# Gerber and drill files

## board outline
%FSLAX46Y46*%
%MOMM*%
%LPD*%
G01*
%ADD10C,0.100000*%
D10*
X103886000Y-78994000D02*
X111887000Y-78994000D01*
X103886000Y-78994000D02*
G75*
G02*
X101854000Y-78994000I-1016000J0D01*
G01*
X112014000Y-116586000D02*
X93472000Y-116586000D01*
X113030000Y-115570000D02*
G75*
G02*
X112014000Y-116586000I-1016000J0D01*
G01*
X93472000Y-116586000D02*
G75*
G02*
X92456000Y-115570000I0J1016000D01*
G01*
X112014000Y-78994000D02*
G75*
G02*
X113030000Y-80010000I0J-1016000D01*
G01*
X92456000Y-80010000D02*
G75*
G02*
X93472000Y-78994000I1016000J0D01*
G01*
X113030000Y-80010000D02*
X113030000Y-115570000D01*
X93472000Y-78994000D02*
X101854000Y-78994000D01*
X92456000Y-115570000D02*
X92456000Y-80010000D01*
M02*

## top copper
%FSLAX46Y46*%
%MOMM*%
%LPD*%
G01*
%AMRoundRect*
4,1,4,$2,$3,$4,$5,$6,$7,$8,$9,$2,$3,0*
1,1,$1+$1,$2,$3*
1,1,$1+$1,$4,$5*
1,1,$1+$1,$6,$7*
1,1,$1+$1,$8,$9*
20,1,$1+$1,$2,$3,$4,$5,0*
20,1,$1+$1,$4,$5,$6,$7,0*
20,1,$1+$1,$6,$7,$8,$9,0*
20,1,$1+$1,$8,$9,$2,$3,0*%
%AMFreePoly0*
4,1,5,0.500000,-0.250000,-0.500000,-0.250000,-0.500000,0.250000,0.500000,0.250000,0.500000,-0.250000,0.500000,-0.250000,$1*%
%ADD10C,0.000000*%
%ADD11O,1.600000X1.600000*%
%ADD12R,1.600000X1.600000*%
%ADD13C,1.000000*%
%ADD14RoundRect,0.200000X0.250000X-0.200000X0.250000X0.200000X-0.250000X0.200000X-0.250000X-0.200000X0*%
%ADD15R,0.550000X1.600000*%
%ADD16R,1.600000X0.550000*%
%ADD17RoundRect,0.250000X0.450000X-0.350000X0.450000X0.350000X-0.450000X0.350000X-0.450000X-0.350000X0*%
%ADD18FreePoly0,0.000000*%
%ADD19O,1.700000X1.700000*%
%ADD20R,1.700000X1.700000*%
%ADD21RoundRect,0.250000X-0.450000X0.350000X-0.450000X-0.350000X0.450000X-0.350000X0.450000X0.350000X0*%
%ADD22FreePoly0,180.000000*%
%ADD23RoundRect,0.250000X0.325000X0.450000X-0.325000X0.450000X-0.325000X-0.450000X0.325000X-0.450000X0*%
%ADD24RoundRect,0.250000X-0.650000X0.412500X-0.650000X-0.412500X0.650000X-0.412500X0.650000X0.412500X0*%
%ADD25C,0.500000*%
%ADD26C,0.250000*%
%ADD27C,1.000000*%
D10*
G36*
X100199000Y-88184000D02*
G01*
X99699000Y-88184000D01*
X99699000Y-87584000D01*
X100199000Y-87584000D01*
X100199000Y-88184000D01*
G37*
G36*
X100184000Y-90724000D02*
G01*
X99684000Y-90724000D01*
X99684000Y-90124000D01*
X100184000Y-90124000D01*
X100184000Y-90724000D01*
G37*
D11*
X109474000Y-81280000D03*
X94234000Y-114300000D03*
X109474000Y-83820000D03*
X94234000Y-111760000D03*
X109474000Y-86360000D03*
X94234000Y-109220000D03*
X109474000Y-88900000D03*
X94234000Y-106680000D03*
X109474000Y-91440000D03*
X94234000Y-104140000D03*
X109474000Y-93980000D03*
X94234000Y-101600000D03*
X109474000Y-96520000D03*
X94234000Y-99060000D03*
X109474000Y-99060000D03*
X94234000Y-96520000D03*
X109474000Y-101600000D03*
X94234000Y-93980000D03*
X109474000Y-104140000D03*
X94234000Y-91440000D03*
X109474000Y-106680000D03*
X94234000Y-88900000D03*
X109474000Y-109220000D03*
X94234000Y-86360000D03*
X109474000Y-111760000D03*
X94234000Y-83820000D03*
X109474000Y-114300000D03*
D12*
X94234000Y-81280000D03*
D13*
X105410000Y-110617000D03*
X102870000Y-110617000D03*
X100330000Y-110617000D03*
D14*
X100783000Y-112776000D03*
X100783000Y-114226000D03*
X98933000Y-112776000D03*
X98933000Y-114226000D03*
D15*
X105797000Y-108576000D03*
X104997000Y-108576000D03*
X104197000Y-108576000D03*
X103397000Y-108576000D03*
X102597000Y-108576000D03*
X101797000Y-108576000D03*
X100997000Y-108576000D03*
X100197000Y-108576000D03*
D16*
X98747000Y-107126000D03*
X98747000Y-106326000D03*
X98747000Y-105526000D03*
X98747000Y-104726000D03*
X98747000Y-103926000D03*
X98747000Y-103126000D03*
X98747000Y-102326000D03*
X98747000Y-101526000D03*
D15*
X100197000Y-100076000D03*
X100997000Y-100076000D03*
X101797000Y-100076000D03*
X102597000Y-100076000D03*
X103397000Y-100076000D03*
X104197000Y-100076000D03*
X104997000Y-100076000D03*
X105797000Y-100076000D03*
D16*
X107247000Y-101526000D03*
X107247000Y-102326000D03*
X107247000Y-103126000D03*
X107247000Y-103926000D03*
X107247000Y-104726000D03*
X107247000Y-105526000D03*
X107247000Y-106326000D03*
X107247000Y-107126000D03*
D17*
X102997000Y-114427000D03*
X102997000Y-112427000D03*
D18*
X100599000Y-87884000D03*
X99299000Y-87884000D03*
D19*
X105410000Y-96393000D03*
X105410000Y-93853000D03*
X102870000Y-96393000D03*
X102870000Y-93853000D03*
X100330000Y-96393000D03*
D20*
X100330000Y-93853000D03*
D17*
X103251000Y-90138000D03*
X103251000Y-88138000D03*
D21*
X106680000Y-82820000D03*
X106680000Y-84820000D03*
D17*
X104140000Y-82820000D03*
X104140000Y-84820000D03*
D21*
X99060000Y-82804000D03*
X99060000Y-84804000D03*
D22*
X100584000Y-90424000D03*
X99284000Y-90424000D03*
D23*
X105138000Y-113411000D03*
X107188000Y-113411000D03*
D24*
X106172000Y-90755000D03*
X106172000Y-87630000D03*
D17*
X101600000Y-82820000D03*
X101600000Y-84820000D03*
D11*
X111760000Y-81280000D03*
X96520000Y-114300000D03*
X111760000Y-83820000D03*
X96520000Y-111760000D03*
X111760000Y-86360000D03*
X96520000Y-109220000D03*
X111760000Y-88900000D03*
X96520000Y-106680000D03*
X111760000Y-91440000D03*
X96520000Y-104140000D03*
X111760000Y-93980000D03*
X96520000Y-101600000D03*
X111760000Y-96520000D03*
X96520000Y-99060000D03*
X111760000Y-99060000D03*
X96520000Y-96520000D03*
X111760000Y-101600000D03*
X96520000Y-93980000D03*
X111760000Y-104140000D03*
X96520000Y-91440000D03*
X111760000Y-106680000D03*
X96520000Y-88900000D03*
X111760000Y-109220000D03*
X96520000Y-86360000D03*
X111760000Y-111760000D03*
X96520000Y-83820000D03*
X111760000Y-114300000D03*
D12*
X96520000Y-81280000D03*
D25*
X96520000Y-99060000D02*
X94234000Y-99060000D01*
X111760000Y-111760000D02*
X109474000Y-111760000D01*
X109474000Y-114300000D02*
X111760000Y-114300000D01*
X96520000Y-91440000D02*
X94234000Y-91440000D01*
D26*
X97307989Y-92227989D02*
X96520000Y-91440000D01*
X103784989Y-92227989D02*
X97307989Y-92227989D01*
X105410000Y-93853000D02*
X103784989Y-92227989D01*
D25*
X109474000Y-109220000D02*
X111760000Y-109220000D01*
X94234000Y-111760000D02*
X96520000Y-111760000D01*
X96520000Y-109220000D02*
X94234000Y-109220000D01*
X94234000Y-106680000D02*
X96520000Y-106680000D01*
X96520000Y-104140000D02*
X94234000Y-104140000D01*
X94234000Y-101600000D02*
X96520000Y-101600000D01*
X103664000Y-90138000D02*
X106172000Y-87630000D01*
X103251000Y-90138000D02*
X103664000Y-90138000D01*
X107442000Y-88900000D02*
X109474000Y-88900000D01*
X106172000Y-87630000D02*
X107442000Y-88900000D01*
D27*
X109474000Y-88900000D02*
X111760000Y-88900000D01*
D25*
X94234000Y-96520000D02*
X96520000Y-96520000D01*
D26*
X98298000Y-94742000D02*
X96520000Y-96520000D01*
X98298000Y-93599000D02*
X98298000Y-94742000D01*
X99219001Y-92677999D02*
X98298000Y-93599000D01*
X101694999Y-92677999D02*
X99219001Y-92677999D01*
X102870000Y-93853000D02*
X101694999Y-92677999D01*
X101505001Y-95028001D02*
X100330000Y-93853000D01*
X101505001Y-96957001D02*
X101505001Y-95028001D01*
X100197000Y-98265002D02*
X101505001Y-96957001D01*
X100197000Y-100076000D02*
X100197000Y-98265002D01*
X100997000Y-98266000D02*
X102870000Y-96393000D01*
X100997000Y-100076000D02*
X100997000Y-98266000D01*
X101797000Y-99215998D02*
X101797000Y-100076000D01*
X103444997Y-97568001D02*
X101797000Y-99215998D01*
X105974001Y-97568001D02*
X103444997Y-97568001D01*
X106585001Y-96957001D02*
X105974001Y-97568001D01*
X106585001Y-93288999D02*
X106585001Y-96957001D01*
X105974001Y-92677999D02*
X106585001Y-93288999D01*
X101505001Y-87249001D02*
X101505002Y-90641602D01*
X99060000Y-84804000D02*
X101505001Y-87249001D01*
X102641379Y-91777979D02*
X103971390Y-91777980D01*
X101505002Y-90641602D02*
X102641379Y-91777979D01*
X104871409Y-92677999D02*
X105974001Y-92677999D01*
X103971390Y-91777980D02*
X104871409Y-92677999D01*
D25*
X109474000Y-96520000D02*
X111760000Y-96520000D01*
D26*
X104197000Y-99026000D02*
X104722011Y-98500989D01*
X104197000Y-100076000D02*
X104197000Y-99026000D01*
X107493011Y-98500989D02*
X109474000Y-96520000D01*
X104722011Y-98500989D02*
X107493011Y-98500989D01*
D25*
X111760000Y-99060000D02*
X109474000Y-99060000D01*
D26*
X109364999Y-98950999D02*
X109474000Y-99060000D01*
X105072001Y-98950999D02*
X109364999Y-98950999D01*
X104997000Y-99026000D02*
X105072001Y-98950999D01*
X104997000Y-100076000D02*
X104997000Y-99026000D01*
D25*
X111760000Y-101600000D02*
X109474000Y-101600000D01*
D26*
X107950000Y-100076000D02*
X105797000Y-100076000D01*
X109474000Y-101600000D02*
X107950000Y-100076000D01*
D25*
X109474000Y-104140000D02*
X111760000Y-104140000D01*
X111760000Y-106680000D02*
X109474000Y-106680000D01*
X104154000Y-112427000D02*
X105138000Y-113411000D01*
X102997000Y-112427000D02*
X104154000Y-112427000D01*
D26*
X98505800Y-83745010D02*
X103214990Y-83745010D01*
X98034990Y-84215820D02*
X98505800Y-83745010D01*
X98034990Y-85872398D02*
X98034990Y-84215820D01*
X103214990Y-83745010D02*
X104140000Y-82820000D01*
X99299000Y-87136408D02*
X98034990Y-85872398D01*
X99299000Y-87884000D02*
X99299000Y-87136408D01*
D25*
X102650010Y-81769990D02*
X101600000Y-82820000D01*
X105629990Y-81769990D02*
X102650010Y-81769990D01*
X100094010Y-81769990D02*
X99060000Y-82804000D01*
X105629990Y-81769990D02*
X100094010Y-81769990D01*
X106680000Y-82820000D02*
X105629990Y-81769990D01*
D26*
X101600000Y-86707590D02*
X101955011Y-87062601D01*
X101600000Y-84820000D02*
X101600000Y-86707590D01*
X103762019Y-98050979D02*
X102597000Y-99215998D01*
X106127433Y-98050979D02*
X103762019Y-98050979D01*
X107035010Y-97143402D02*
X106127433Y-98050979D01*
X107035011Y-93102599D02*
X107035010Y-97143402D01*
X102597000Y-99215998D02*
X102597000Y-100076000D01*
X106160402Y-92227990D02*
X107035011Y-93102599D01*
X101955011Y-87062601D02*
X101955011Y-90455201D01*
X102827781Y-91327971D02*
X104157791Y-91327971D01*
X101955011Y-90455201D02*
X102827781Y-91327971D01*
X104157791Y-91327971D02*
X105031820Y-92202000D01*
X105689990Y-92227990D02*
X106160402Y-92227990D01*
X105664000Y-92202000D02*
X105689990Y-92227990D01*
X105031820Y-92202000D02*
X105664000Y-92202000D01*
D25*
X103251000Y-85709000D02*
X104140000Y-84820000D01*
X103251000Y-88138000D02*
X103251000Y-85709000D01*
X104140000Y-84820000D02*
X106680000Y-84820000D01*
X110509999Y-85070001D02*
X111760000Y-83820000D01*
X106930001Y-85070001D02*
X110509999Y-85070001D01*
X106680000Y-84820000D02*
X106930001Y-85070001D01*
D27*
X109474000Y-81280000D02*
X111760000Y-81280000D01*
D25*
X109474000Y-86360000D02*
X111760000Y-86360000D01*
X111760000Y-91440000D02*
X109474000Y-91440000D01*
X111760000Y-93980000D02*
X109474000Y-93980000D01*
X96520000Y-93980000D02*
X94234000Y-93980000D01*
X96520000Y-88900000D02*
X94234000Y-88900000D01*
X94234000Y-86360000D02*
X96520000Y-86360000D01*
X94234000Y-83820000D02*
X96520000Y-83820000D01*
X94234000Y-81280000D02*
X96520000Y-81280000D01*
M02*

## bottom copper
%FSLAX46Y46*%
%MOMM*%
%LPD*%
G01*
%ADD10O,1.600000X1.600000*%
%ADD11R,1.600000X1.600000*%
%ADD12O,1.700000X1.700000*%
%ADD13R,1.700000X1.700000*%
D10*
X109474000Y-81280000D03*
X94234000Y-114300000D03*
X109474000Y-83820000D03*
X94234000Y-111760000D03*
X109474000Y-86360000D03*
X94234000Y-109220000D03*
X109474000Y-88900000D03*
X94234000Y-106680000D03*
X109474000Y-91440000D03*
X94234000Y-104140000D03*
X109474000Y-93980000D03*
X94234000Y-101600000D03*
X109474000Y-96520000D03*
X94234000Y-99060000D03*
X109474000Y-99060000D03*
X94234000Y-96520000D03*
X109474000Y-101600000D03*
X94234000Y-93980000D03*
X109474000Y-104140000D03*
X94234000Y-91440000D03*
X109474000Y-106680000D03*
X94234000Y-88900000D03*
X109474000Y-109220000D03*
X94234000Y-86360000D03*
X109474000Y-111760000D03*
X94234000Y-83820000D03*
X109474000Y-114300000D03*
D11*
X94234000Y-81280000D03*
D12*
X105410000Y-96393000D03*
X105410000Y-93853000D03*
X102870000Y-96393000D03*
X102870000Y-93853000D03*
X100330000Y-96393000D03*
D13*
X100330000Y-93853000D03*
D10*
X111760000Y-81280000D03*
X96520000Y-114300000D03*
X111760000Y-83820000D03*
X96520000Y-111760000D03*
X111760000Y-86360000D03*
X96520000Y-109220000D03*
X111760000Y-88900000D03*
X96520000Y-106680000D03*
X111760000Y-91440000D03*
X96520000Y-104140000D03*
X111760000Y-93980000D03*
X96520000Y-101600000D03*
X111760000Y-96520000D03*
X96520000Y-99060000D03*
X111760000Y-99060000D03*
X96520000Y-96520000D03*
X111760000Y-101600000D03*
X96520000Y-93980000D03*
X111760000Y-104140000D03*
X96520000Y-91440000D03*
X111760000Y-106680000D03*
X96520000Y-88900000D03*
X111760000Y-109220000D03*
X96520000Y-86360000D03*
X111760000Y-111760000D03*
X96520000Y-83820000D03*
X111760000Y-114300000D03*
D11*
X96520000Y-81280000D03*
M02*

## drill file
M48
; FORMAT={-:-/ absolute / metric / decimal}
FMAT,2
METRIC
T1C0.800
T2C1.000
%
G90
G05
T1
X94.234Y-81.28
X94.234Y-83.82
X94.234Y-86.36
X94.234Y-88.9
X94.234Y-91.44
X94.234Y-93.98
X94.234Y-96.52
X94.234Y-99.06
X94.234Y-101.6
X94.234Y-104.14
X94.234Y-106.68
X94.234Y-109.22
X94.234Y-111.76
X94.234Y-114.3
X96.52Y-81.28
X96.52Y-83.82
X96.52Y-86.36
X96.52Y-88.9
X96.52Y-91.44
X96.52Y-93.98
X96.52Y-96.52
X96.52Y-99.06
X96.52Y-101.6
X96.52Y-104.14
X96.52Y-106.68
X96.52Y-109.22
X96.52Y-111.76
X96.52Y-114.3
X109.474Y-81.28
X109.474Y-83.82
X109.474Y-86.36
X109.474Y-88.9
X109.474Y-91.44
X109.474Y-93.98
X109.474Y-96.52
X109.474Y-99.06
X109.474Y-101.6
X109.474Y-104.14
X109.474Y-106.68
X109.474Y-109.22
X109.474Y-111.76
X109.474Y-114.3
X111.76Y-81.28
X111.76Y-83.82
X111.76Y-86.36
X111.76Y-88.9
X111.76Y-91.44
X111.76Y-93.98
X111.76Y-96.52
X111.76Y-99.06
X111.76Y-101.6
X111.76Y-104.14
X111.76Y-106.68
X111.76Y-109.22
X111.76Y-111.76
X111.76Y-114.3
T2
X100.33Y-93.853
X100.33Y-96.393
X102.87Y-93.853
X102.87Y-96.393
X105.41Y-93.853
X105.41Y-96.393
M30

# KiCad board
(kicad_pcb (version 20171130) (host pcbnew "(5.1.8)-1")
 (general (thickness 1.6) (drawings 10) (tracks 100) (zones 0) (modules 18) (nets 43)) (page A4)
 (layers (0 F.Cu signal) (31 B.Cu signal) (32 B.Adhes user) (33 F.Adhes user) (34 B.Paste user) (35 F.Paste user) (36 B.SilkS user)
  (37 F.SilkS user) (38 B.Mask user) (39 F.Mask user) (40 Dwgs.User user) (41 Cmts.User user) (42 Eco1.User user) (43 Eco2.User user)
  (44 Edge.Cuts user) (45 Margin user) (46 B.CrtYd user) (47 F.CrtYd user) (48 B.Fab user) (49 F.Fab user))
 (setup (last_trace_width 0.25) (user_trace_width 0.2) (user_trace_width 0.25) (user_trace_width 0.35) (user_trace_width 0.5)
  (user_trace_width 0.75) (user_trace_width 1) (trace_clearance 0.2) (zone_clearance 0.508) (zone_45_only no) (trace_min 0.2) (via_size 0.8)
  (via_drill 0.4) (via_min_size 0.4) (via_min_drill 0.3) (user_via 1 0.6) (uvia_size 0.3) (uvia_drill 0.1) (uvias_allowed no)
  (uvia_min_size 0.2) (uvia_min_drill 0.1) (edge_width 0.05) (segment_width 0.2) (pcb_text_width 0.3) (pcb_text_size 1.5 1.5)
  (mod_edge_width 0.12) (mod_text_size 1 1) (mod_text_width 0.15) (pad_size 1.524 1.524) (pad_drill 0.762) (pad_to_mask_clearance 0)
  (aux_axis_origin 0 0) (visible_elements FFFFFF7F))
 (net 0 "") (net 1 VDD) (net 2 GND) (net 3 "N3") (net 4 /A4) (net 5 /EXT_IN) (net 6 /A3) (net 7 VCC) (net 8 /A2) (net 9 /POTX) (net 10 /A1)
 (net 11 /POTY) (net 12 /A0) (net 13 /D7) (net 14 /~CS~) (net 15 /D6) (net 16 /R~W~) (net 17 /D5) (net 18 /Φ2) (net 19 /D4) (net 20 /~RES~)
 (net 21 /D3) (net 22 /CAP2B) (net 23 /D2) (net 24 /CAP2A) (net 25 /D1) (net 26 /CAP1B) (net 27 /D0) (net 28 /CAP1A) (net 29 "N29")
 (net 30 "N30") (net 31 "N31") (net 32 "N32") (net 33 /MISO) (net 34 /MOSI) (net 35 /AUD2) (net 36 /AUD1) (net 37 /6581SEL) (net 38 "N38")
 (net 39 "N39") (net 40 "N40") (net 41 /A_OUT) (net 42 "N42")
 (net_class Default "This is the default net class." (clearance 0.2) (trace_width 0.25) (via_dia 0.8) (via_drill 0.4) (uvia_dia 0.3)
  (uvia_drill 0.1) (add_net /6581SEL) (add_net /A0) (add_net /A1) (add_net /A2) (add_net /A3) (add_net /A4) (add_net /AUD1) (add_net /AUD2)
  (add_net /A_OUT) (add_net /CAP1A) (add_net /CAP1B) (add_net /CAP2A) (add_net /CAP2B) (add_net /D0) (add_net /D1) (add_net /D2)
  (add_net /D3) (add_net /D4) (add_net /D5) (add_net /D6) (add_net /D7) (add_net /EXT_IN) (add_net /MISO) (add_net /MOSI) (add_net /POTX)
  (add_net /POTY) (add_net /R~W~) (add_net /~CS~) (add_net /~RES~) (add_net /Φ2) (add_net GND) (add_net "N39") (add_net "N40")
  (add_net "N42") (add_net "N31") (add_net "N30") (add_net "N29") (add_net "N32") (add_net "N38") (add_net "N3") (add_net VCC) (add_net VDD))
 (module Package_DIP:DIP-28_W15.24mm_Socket (layer F.Cu) (at 94.234 81.28)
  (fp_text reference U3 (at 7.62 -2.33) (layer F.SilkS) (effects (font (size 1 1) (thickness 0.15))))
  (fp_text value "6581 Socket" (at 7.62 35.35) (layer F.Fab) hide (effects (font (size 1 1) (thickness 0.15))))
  (pad 28 thru_hole oval (at 15.24 0) (size 1.6 1.6) (drill 0.8) (layers *.Cu *.Mask) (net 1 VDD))
  (pad 14 thru_hole oval (at 0 33.02) (size 1.6 1.6) (drill 0.8) (layers *.Cu *.Mask) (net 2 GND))
  (pad 27 thru_hole oval (at 15.24 2.54) (size 1.6 1.6) (drill 0.8) (layers *.Cu *.Mask) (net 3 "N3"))
  (pad 13 thru_hole oval (at 0 30.48) (size 1.6 1.6) (drill 0.8) (layers *.Cu *.Mask) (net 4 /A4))
  (pad 26 thru_hole oval (at 15.24 5.08) (size 1.6 1.6) (drill 0.8) (layers *.Cu *.Mask) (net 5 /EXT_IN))
  (pad 12 thru_hole oval (at 0 27.94) (size 1.6 1.6) (drill 0.8) (layers *.Cu *.Mask) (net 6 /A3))
  (pad 25 thru_hole oval (at 15.24 7.62) (size 1.6 1.6) (drill 0.8) (layers *.Cu *.Mask) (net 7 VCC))
  (pad 11 thru_hole oval (at 0 25.4) (size 1.6 1.6) (drill 0.8) (layers *.Cu *.Mask) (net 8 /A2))
  (pad 24 thru_hole oval (at 15.24 10.16) (size 1.6 1.6) (drill 0.8) (layers *.Cu *.Mask) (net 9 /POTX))
  (pad 10 thru_hole oval (at 0 22.86) (size 1.6 1.6) (drill 0.8) (layers *.Cu *.Mask) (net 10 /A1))
  (pad 23 thru_hole oval (at 15.24 12.7) (size 1.6 1.6) (drill 0.8) (layers *.Cu *.Mask) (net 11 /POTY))
  (pad 9 thru_hole oval (at 0 20.32) (size 1.6 1.6) (drill 0.8) (layers *.Cu *.Mask) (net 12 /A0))
  (pad 22 thru_hole oval (at 15.24 15.24) (size 1.6 1.6) (drill 0.8) (layers *.Cu *.Mask) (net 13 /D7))
  (pad 8 thru_hole oval (at 0 17.78) (size 1.6 1.6) (drill 0.8) (layers *.Cu *.Mask) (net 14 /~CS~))
  (pad 21 thru_hole oval (at 15.24 17.78) (size 1.6 1.6) (drill 0.8) (layers *.Cu *.Mask) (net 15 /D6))
  (pad 7 thru_hole oval (at 0 15.24) (size 1.6 1.6) (drill 0.8) (layers *.Cu *.Mask) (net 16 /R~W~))
  (pad 20 thru_hole oval (at 15.24 20.32) (size 1.6 1.6) (drill 0.8) (layers *.Cu *.Mask) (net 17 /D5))
  (pad 6 thru_hole oval (at 0 12.7) (size 1.6 1.6) (drill 0.8) (layers *.Cu *.Mask) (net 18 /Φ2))
  (pad 19 thru_hole oval (at 15.24 22.86) (size 1.6 1.6) (drill 0.8) (layers *.Cu *.Mask) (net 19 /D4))
  (pad 5 thru_hole oval (at 0 10.16) (size 1.6 1.6) (drill 0.8) (layers *.Cu *.Mask) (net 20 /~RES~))
  (pad 18 thru_hole oval (at 15.24 25.4) (size 1.6 1.6) (drill 0.8) (layers *.Cu *.Mask) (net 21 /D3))
  (pad 4 thru_hole oval (at 0 7.62) (size 1.6 1.6) (drill 0.8) (layers *.Cu *.Mask) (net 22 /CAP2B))
  (pad 17 thru_hole oval (at 15.24 27.94) (size 1.6 1.6) (drill 0.8) (layers *.Cu *.Mask) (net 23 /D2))
  (pad 3 thru_hole oval (at 0 5.08) (size 1.6 1.6) (drill 0.8) (layers *.Cu *.Mask) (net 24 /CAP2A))
  (pad 16 thru_hole oval (at 15.24 30.48) (size 1.6 1.6) (drill 0.8) (layers *.Cu *.Mask) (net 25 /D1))
  (pad 2 thru_hole oval (at 0 2.54) (size 1.6 1.6) (drill 0.8) (layers *.Cu *.Mask) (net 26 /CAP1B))
  (pad 15 thru_hole oval (at 15.24 33.02) (size 1.6 1.6) (drill 0.8) (layers *.Cu *.Mask) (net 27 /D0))
  (pad 1 thru_hole rect (at 0 0) (size 1.6 1.6) (drill 0.8) (layers *.Cu *.Mask) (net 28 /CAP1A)))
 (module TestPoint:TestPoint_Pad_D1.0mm (layer F.Cu) (at 105.41 110.617)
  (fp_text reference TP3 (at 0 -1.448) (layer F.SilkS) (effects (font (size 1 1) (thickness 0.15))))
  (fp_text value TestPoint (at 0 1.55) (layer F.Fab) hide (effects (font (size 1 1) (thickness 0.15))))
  (pad 1 smd circle (at 0 0) (size 1 1) (layers F.Cu F.Mask) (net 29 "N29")))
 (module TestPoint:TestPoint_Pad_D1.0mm (layer F.Cu) (at 102.87 110.617)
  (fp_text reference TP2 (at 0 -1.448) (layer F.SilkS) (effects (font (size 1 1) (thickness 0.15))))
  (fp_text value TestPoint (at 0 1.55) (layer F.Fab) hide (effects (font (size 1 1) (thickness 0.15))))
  (pad 1 smd circle (at 0 0) (size 1 1) (layers F.Cu F.Mask) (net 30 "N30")))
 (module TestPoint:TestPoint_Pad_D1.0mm (layer F.Cu) (at 100.33 110.617)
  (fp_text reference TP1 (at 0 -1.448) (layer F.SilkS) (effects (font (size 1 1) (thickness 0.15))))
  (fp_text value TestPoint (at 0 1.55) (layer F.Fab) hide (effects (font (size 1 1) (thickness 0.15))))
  (pad 1 smd circle (at 0 0) (size 1 1) (layers F.Cu F.Mask) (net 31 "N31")))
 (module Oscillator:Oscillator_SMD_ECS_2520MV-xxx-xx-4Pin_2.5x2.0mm (layer F.Cu) (at 99.858 113.501 90)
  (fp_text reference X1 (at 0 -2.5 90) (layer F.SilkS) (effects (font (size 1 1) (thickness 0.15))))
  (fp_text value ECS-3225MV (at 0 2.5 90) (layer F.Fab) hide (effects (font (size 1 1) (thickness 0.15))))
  (pad 3 smd roundrect (at 0.725 0.925 90) (size 0.8 0.9) (layers F.Cu F.Paste F.Mask) (roundrect_rratio 0.25) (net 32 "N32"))
  (pad 2 smd roundrect (at -0.725 0.925 90) (size 0.8 0.9) (layers F.Cu F.Paste F.Mask) (roundrect_rratio 0.25) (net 2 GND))
  (pad 4 smd roundrect (at 0.725 -0.925 90) (size 0.8 0.9) (layers F.Cu F.Paste F.Mask) (roundrect_rratio 0.25) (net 7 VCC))
  (pad 1 smd roundrect (at -0.725 -0.925 90) (size 0.8 0.9) (layers F.Cu F.Paste F.Mask) (roundrect_rratio 0.25) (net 7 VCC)))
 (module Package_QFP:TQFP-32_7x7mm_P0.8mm (layer F.Cu) (at 102.997 104.326 180)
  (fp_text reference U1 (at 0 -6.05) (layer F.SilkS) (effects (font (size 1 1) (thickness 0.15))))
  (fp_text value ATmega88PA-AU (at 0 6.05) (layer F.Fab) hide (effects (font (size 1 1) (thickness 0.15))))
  (pad 32 smd rect (at -2.8 -4.25 270) (size 1.6 0.55) (layers F.Cu F.Paste F.Mask) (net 14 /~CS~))
  (pad 31 smd rect (at -2 -4.25 270) (size 1.6 0.55) (layers F.Cu F.Paste F.Mask) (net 25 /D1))
  (pad 30 smd rect (at -1.2 -4.25 270) (size 1.6 0.55) (layers F.Cu F.Paste F.Mask) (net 27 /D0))
  (pad 29 smd rect (at -0.4 -4.25 270) (size 1.6 0.55) (layers F.Cu F.Paste F.Mask) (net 20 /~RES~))
  (pad 28 smd rect (at 0.4 -4.25 270) (size 1.6 0.55) (layers F.Cu F.Paste F.Mask) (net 23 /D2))
  (pad 27 smd rect (at 1.2 -4.25 270) (size 1.6 0.55) (layers F.Cu F.Paste F.Mask) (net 4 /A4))
  (pad 26 smd rect (at 2 -4.25 270) (size 1.6 0.55) (layers F.Cu F.Paste F.Mask) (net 6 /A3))
  (pad 25 smd rect (at 2.8 -4.25 270) (size 1.6 0.55) (layers F.Cu F.Paste F.Mask) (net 8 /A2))
  (pad 24 smd rect (at 4.25 -2.8 180) (size 1.6 0.55) (layers F.Cu F.Paste F.Mask) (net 10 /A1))
  (pad 23 smd rect (at 4.25 -2 180) (size 1.6 0.55) (layers F.Cu F.Paste F.Mask) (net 12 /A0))
  (pad 22 smd rect (at 4.25 -1.2 180) (size 1.6 0.55) (layers F.Cu F.Paste F.Mask) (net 30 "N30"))
  (pad 21 smd rect (at 4.25 -0.4 180) (size 1.6 0.55) (layers F.Cu F.Paste F.Mask) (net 2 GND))
  (pad 20 smd rect (at 4.25 0.4 180) (size 1.6 0.55) (layers F.Cu F.Paste F.Mask) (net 29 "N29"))
  (pad 19 smd rect (at 4.25 1.2 180) (size 1.6 0.55) (layers F.Cu F.Paste F.Mask) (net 31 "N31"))
  (pad 18 smd rect (at 4.25 2 180) (size 1.6 0.55) (layers F.Cu F.Paste F.Mask) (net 7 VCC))
  (pad 17 smd rect (at 4.25 2.8 180) (size 1.6 0.55) (layers F.Cu F.Paste F.Mask) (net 16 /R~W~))
  (pad 16 smd rect (at 2.8 4.25 270) (size 1.6 0.55) (layers F.Cu F.Paste F.Mask) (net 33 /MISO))
  (pad 15 smd rect (at 2 4.25 270) (size 1.6 0.55) (layers F.Cu F.Paste F.Mask) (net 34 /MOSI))
  (pad 14 smd rect (at 1.2 4.25 270) (size 1.6 0.55) (layers F.Cu F.Paste F.Mask) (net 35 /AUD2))
  (pad 13 smd rect (at 0.4 4.25 270) (size 1.6 0.55) (layers F.Cu F.Paste F.Mask) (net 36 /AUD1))
  (pad 12 smd rect (at -0.4 4.25 270) (size 1.6 0.55) (layers F.Cu F.Paste F.Mask) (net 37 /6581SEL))
  (pad 11 smd rect (at -1.2 4.25 270) (size 1.6 0.55) (layers F.Cu F.Paste F.Mask) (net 13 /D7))
  (pad 10 smd rect (at -2 4.25 270) (size 1.6 0.55) (layers F.Cu F.Paste F.Mask) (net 15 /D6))
  (pad 9 smd rect (at -2.8 4.25 270) (size 1.6 0.55) (layers F.Cu F.Paste F.Mask) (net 17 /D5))
  (pad 8 smd rect (at -4.25 2.8 180) (size 1.6 0.55) (layers F.Cu F.Paste F.Mask) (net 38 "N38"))
  (pad 7 smd rect (at -4.25 2 180) (size 1.6 0.55) (layers F.Cu F.Paste F.Mask) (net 32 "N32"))
  (pad 6 smd rect (at -4.25 1.2 180) (size 1.6 0.55) (layers F.Cu F.Paste F.Mask) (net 7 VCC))
  (pad 5 smd rect (at -4.25 0.4 180) (size 1.6 0.55) (layers F.Cu F.Paste F.Mask) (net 2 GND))
  (pad 4 smd rect (at -4.25 -0.4 180) (size 1.6 0.55) (layers F.Cu F.Paste F.Mask) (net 7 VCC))
  (pad 3 smd rect (at -4.25 -1.2 180) (size 1.6 0.55) (layers F.Cu F.Paste F.Mask) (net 2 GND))
  (pad 2 smd rect (at -4.25 -2 180) (size 1.6 0.55) (layers F.Cu F.Paste F.Mask) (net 19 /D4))
  (pad 1 smd rect (at -4.25 -2.8 180) (size 1.6 0.55) (layers F.Cu F.Paste F.Mask) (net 21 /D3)))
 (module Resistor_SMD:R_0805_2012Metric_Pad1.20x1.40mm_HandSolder (layer F.Cu) (at 102.997 113.427 90)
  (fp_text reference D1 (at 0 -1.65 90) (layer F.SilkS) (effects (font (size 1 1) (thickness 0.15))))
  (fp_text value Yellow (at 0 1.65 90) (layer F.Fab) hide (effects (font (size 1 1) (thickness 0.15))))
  (pad 1 smd roundrect (at -1 0 90) (size 1.2 1.4) (layers F.Cu F.Paste F.Mask) (roundrect_rratio 0.208333) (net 2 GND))
  (pad 2 smd roundrect (at 1 0 90) (size 1.2 1.4) (layers F.Cu F.Paste F.Mask) (roundrect_rratio 0.208333) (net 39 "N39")))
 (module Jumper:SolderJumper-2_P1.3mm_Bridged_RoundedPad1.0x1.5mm (layer F.Cu) (at 99.949 87.884)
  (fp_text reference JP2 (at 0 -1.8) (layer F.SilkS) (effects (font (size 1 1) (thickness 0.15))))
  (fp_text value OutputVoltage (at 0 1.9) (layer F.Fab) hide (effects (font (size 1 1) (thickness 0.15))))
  (fp_poly (pts (xy 0.25 -0.3) (xy -0.25 -0.3) (xy -0.25 0.3) (xy 0.25 0.3)) (layer F.Cu) (width 0))
  (pad 2 smd custom (at 0.65 0) (size 1 0.5) (layers F.Cu F.Mask) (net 2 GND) (zone_connect 2) (options (clearance outline) (anchor rect))
   (primitives))
  (pad 1 smd custom (at -0.65 0) (size 1 0.5) (layers F.Cu F.Mask) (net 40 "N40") (zone_connect 2)
   (options (clearance outline) (anchor rect)) (primitives)))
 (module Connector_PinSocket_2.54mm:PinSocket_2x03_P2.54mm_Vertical (layer F.Cu) (at 100.33 93.853 90)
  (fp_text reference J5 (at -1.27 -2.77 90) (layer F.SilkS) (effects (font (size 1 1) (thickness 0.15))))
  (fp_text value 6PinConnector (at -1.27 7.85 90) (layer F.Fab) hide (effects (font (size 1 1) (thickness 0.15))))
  (pad 6 thru_hole oval (at -2.54 5.08 90) (size 1.7 1.7) (drill 1) (layers *.Cu *.Mask) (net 2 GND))
  (pad 5 thru_hole oval (at 0 5.08 90) (size 1.7 1.7) (drill 1) (layers *.Cu *.Mask) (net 20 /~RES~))
  (pad 4 thru_hole oval (at -2.54 2.54 90) (size 1.7 1.7) (drill 1) (layers *.Cu *.Mask) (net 34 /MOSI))
  (pad 3 thru_hole oval (at 0 2.54 90) (size 1.7 1.7) (drill 1) (layers *.Cu *.Mask) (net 16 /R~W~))
  (pad 2 thru_hole oval (at -2.54 0 90) (size 1.7 1.7) (drill 1) (layers *.Cu *.Mask) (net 7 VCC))
  (pad 1 thru_hole rect (at 0 0 90) (size 1.7 1.7) (drill 1) (layers *.Cu *.Mask) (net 33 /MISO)))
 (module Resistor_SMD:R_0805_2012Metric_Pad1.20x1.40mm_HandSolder (layer F.Cu) (at 103.251 89.138 90)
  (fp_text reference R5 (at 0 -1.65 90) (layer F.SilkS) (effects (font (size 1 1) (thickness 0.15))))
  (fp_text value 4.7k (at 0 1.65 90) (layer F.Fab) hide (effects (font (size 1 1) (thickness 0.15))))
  (pad 1 smd roundrect (at -1 0 90) (size 1.2 1.4) (layers F.Cu F.Paste F.Mask) (roundrect_rratio 0.208333) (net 7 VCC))
  (pad 2 smd roundrect (at 1 0 90) (size 1.2 1.4) (layers F.Cu F.Paste F.Mask) (roundrect_rratio 0.208333) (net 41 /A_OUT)))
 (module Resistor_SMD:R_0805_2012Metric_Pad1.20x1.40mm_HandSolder (layer F.Cu) (at 106.68 83.82 270)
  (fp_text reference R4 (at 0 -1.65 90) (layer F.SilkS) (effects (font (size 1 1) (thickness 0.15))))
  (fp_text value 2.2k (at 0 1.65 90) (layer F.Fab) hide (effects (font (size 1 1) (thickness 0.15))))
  (pad 1 smd roundrect (at -1 0 270) (size 1.2 1.4) (layers F.Cu F.Paste F.Mask) (roundrect_rratio 0.208333) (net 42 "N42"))
  (pad 2 smd roundrect (at 1 0 270) (size 1.2 1.4) (layers F.Cu F.Paste F.Mask) (roundrect_rratio 0.208333) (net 41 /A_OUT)))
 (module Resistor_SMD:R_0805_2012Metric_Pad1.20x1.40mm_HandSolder (layer F.Cu) (at 104.14 83.82 90)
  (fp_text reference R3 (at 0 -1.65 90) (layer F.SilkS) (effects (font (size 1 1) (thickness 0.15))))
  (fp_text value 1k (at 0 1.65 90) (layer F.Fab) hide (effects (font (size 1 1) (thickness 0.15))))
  (pad 2 smd roundrect (at 1 0 90) (size 1.2 1.4) (layers F.Cu F.Paste F.Mask) (roundrect_rratio 0.208333) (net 40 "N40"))
  (pad 1 smd roundrect (at -1 0 90) (size 1.2 1.4) (layers F.Cu F.Paste F.Mask) (roundrect_rratio 0.208333) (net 41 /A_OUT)))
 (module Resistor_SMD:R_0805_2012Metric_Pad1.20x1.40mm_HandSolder (layer F.Cu) (at 99.06 83.804 270)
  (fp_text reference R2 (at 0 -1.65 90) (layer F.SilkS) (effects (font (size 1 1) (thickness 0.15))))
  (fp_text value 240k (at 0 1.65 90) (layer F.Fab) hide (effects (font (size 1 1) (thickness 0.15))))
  (pad 1 smd roundrect (at -1 0 270) (size 1.2 1.4) (layers F.Cu F.Paste F.Mask) (roundrect_rratio 0.208333) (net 42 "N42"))
  (pad 2 smd roundrect (at 1 0 270) (size 1.2 1.4) (layers F.Cu F.Paste F.Mask) (roundrect_rratio 0.208333) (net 35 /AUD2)))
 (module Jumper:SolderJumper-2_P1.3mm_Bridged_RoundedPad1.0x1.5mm (layer F.Cu) (at 99.934 90.424 180)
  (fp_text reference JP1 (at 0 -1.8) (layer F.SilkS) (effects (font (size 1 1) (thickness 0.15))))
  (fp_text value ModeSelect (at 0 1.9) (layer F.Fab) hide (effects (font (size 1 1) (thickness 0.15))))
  (fp_poly (pts (xy 0.25 -0.3) (xy -0.25 -0.3) (xy -0.25 0.3) (xy 0.25 0.3)) (layer F.Cu) (width 0))
  (pad 1 smd custom (at -0.65 0 180) (size 1 0.5) (layers F.Cu F.Mask) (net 37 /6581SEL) (zone_connect 2)
   (options (clearance outline) (anchor rect)) (primitives))
  (pad 2 smd custom (at 0.65 0 180) (size 1 0.5) (layers F.Cu F.Mask) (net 2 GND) (zone_connect 2)
   (options (clearance outline) (anchor rect)) (primitives)))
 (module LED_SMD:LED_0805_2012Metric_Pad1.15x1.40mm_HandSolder (layer F.Cu) (at 106.163 113.411 180)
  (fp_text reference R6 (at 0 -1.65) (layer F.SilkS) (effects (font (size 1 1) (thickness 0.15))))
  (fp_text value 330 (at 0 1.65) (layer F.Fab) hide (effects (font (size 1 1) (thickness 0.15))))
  (pad 2 smd roundrect (at 1.025 0 180) (size 1.15 1.4) (layers F.Cu F.Paste F.Mask) (roundrect_rratio 0.217391) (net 39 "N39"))
  (pad 1 smd roundrect (at -1.025 0 180) (size 1.15 1.4) (layers F.Cu F.Paste F.Mask) (roundrect_rratio 0.217391) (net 7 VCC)))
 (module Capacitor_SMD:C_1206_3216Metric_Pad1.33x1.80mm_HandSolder (layer F.Cu) (at 106.172 89.1925 270)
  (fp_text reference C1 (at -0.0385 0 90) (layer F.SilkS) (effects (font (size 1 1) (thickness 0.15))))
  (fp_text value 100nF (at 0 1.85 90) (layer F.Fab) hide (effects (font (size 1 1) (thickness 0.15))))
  (pad 2 smd roundrect (at 1.5625 0 270) (size 1.325 1.8) (layers F.Cu F.Paste F.Mask) (roundrect_rratio 0.188679) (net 2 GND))
  (pad 1 smd roundrect (at -1.5625 0 270) (size 1.325 1.8) (layers F.Cu F.Paste F.Mask) (roundrect_rratio 0.188679) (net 7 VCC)))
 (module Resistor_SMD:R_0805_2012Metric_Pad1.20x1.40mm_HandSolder (layer F.Cu) (at 101.6 83.82 90)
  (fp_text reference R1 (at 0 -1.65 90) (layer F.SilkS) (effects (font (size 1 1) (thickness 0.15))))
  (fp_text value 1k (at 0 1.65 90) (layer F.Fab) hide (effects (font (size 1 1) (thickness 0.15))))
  (pad 2 smd roundrect (at 1 0 90) (size 1.2 1.4) (layers F.Cu F.Paste F.Mask) (roundrect_rratio 0.208333) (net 42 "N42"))
  (pad 1 smd roundrect (at -1 0 90) (size 1.2 1.4) (layers F.Cu F.Paste F.Mask) (roundrect_rratio 0.208333) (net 36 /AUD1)))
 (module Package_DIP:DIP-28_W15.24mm (layer F.Cu) (at 96.52 81.28)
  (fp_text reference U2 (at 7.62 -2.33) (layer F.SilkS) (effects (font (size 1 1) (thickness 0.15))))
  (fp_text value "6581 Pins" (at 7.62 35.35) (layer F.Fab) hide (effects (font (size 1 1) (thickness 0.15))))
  (pad 28 thru_hole oval (at 15.24 0) (size 1.6 1.6) (drill 0.8) (layers *.Cu *.Mask) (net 1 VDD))
  (pad 14 thru_hole oval (at 0 33.02) (size 1.6 1.6) (drill 0.8) (layers *.Cu *.Mask) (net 2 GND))
  (pad 27 thru_hole oval (at 15.24 2.54) (size 1.6 1.6) (drill 0.8) (layers *.Cu *.Mask) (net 41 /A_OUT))
  (pad 13 thru_hole oval (at 0 30.48) (size 1.6 1.6) (drill 0.8) (layers *.Cu *.Mask) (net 4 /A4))
  (pad 26 thru_hole oval (at 15.24 5.08) (size 1.6 1.6) (drill 0.8) (layers *.Cu *.Mask) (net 5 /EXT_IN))
  (pad 12 thru_hole oval (at 0 27.94) (size 1.6 1.6) (drill 0.8) (layers *.Cu *.Mask) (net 6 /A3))
  (pad 25 thru_hole oval (at 15.24 7.62) (size 1.6 1.6) (drill 0.8) (layers *.Cu *.Mask) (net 7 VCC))
  (pad 11 thru_hole oval (at 0 25.4) (size 1.6 1.6) (drill 0.8) (layers *.Cu *.Mask) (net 8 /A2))
  (pad 24 thru_hole oval (at 15.24 10.16) (size 1.6 1.6) (drill 0.8) (layers *.Cu *.Mask) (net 9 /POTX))
  (pad 10 thru_hole oval (at 0 22.86) (size 1.6 1.6) (drill 0.8) (layers *.Cu *.Mask) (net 10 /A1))
  (pad 23 thru_hole oval (at 15.24 12.7) (size 1.6 1.6) (drill 0.8) (layers *.Cu *.Mask) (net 11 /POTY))
  (pad 9 thru_hole oval (at 0 20.32) (size 1.6 1.6) (drill 0.8) (layers *.Cu *.Mask) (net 12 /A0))
  (pad 22 thru_hole oval (at 15.24 15.24) (size 1.6 1.6) (drill 0.8) (layers *.Cu *.Mask) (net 13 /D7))
  (pad 8 thru_hole oval (at 0 17.78) (size 1.6 1.6) (drill 0.8) (layers *.Cu *.Mask) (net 14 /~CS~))
  (pad 21 thru_hole oval (at 15.24 17.78) (size 1.6 1.6) (drill 0.8) (layers *.Cu *.Mask) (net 15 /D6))
  (pad 7 thru_hole oval (at 0 15.24) (size 1.6 1.6) (drill 0.8) (layers *.Cu *.Mask) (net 16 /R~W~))
  (pad 20 thru_hole oval (at 15.24 20.32) (size 1.6 1.6) (drill 0.8) (layers *.Cu *.Mask) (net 17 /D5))
  (pad 6 thru_hole oval (at 0 12.7) (size 1.6 1.6) (drill 0.8) (layers *.Cu *.Mask) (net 18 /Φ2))
  (pad 19 thru_hole oval (at 15.24 22.86) (size 1.6 1.6) (drill 0.8) (layers *.Cu *.Mask) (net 19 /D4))
  (pad 5 thru_hole oval (at 0 10.16) (size 1.6 1.6) (drill 0.8) (layers *.Cu *.Mask) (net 20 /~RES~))
  (pad 18 thru_hole oval (at 15.24 25.4) (size 1.6 1.6) (drill 0.8) (layers *.Cu *.Mask) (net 21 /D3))
  (pad 4 thru_hole oval (at 0 7.62) (size 1.6 1.6) (drill 0.8) (layers *.Cu *.Mask) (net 22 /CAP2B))
  (pad 17 thru_hole oval (at 15.24 27.94) (size 1.6 1.6) (drill 0.8) (layers *.Cu *.Mask) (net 23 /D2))
  (pad 3 thru_hole oval (at 0 5.08) (size 1.6 1.6) (drill 0.8) (layers *.Cu *.Mask) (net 24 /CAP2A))
  (pad 16 thru_hole oval (at 15.24 30.48) (size 1.6 1.6) (drill 0.8) (layers *.Cu *.Mask) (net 25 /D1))
  (pad 2 thru_hole oval (at 0 2.54) (size 1.6 1.6) (drill 0.8) (layers *.Cu *.Mask) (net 26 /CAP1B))
  (pad 15 thru_hole oval (at 15.24 33.02) (size 1.6 1.6) (drill 0.8) (layers *.Cu *.Mask) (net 27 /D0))
  (pad 1 thru_hole rect (at 0 0) (size 1.6 1.6) (drill 0.8) (layers *.Cu *.Mask) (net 28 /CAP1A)))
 (gr_line (start 103.886 78.994) (end 111.887 78.994) (layer Edge.Cuts) (width 0.1))
 (gr_arc (start 102.87 78.994) (end 101.854 78.994) (angle -180) (layer Edge.Cuts) (width 0.1))
 (gr_line (start 112.014 116.586) (end 93.472 116.586) (layer Edge.Cuts) (width 0.1))
 (gr_arc (start 112.014 115.57) (end 112.014 116.586) (angle -90) (layer Edge.Cuts) (width 0.1))
 (gr_arc (start 93.472 115.57) (end 92.456 115.57) (angle -90) (layer Edge.Cuts) (width 0.1))
 (gr_arc (start 112.014 80.01) (end 113.03 80.01) (angle -90) (layer Edge.Cuts) (width 0.1))
 (gr_arc (start 93.472 80.01) (end 93.472 78.994) (angle -90) (layer Edge.Cuts) (width 0.1))
 (gr_line (start 113.03 80.01) (end 113.03 115.57) (layer Edge.Cuts) (width 0.1))
 (gr_line (start 93.472 78.994) (end 101.854 78.994) (layer Edge.Cuts) (width 0.1))
 (gr_line (start 92.456 115.57) (end 92.456 80.01) (layer Edge.Cuts) (width 0.1))
 (segment (start 96.52 99.06) (end 94.234 99.06) (width 0.5) (layer F.Cu) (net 14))
 (segment (start 111.76 111.76) (end 109.474 111.76) (width 0.5) (layer F.Cu) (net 25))
 (segment (start 109.474 114.3) (end 111.76 114.3) (width 0.5) (layer F.Cu) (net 27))
 (segment (start 96.52 91.44) (end 94.234 91.44) (width 0.5) (layer F.Cu) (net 20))
 (segment (start 97.307989 92.227989) (end 96.52 91.44) (width 0.25) (layer F.Cu) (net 20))
 (segment (start 103.784989 92.227989) (end 97.307989 92.227989) (width 0.25) (layer F.Cu) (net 20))
 (segment (start 105.41 93.853) (end 103.784989 92.227989) (width 0.25) (layer F.Cu) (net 20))
 (segment (start 109.474 109.22) (end 111.76 109.22) (width 0.5) (layer F.Cu) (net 23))
 (segment (start 94.234 111.76) (end 96.52 111.76) (width 0.5) (layer F.Cu) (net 4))
 (segment (start 96.52 109.22) (end 94.234 109.22) (width 0.5) (layer F.Cu) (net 6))
 (segment (start 94.234 106.68) (end 96.52 106.68) (width 0.5) (layer F.Cu) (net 8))
 (segment (start 96.52 104.14) (end 94.234 104.14) (width 0.5) (layer F.Cu) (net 10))
 (segment (start 94.234 101.6) (end 96.52 101.6) (width 0.5) (layer F.Cu) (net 12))
 (segment (start 103.664 90.138) (end 106.172 87.63) (width 0.5) (layer F.Cu) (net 7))
 (segment (start 103.251 90.138) (end 103.664 90.138) (width 0.5) (layer F.Cu) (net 7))
 (segment (start 107.442 88.9) (end 109.474 88.9) (width 0.5) (layer F.Cu) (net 7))
 (segment (start 106.172 87.63) (end 107.442 88.9) (width 0.5) (layer F.Cu) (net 7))
 (segment (start 109.474 88.9) (end 111.76 88.9) (width 1) (layer F.Cu) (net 7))
 (segment (start 94.234 96.52) (end 96.52 96.52) (width 0.5) (layer F.Cu) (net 16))
 (segment (start 98.298 94.742) (end 96.52 96.52) (width 0.25) (layer F.Cu) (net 16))
 (segment (start 98.298 93.599) (end 98.298 94.742) (width 0.25) (layer F.Cu) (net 16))
 (segment (start 99.219001 92.677999) (end 98.298 93.599) (width 0.25) (layer F.Cu) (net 16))
 (segment (start 101.694999 92.677999) (end 99.219001 92.677999) (width 0.25) (layer F.Cu) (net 16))
 (segment (start 102.87 93.853) (end 101.694999 92.677999) (width 0.25) (layer F.Cu) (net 16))
 (segment (start 101.505001 95.028001) (end 100.33 93.853) (width 0.25) (layer F.Cu) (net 33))
 (segment (start 101.505001 96.957001) (end 101.505001 95.028001) (width 0.25) (layer F.Cu) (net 33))
 (segment (start 100.197 98.265002) (end 101.505001 96.957001) (width 0.25) (layer F.Cu) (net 33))
 (segment (start 100.197 100.076) (end 100.197 98.265002) (width 0.25) (layer F.Cu) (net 33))
 (segment (start 100.997 98.266) (end 102.87 96.393) (width 0.25) (layer F.Cu) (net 34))
 (segment (start 100.997 100.076) (end 100.997 98.266) (width 0.25) (layer F.Cu) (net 34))
 (segment (start 101.797 99.215998) (end 101.797 100.076) (width 0.25) (layer F.Cu) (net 35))
 (segment (start 103.444997 97.568001) (end 101.797 99.215998) (width 0.25) (layer F.Cu) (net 35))
 (segment (start 105.974001 97.568001) (end 103.444997 97.568001) (width 0.25) (layer F.Cu) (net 35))
 (segment (start 106.585001 96.957001) (end 105.974001 97.568001) (width 0.25) (layer F.Cu) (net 35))
 (segment (start 106.585001 93.288999) (end 106.585001 96.957001) (width 0.25) (layer F.Cu) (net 35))
 (segment (start 105.974001 92.677999) (end 106.585001 93.288999) (width 0.25) (layer F.Cu) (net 35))
 (segment (start 101.505001 87.249001) (end 101.505002 90.641602) (width 0.25) (layer F.Cu) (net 35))
 (segment (start 99.06 84.804) (end 101.505001 87.249001) (width 0.25) (layer F.Cu) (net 35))
 (segment (start 102.641379 91.777979) (end 103.97139 91.77798) (width 0.25) (layer F.Cu) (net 35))
 (segment (start 101.505002 90.641602) (end 102.641379 91.777979) (width 0.25) (layer F.Cu) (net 35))
 (segment (start 104.871409 92.677999) (end 105.974001 92.677999) (width 0.25) (layer F.Cu) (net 35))
 (segment (start 103.97139 91.77798) (end 104.871409 92.677999) (width 0.25) (layer F.Cu) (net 35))
 (segment (start 109.474 96.52) (end 111.76 96.52) (width 0.5) (layer F.Cu) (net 13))
 (segment (start 104.197 99.026) (end 104.722011 98.500989) (width 0.25) (layer F.Cu) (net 13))
 (segment (start 104.197 100.076) (end 104.197 99.026) (width 0.25) (layer F.Cu) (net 13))
 (segment (start 107.493011 98.500989) (end 109.474 96.52) (width 0.25) (layer F.Cu) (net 13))
 (segment (start 104.722011 98.500989) (end 107.493011 98.500989) (width 0.25) (layer F.Cu) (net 13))
 (segment (start 111.76 99.06) (end 109.474 99.06) (width 0.5) (layer F.Cu) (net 15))
 (segment (start 109.364999 98.950999) (end 109.474 99.06) (width 0.25) (layer F.Cu) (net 15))
 (segment (start 105.072001 98.950999) (end 109.364999 98.950999) (width 0.25) (layer F.Cu) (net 15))
 (segment (start 104.997 99.026) (end 105.072001 98.950999) (width 0.25) (layer F.Cu) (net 15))
 (segment (start 104.997 100.076) (end 104.997 99.026) (width 0.25) (layer F.Cu) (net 15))
 (segment (start 111.76 101.6) (end 109.474 101.6) (width 0.5) (layer F.Cu) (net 17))
 (segment (start 107.95 100.076) (end 105.797 100.076) (width 0.25) (layer F.Cu) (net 17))
 (segment (start 109.474 101.6) (end 107.95 100.076) (width 0.25) (layer F.Cu) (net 17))
 (segment (start 109.474 104.14) (end 111.76 104.14) (width 0.5) (layer F.Cu) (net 19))
 (segment (start 111.76 106.68) (end 109.474 106.68) (width 0.5) (layer F.Cu) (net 21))
 (segment (start 104.154 112.427) (end 105.138 113.411) (width 0.5) (layer F.Cu) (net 39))
 (segment (start 102.997 112.427) (end 104.154 112.427) (width 0.5) (layer F.Cu) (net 39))
 (segment (start 98.5058 83.74501) (end 103.21499 83.74501) (width 0.25) (layer F.Cu) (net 40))
 (segment (start 98.03499 84.21582) (end 98.5058 83.74501) (width 0.25) (layer F.Cu) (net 40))
 (segment (start 98.03499 85.872398) (end 98.03499 84.21582) (width 0.25) (layer F.Cu) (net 40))
 (segment (start 103.21499 83.74501) (end 104.14 82.82) (width 0.25) (layer F.Cu) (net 40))
 (segment (start 99.299 87.136408) (end 98.03499 85.872398) (width 0.25) (layer F.Cu) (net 40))
 (segment (start 99.299 87.884) (end 99.299 87.136408) (width 0.25) (layer F.Cu) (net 40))
 (segment (start 102.65001 81.76999) (end 101.6 82.82) (width 0.5) (layer F.Cu) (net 42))
 (segment (start 105.62999 81.76999) (end 102.65001 81.76999) (width 0.5) (layer F.Cu) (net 42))
 (segment (start 100.09401 81.76999) (end 99.06 82.804) (width 0.5) (layer F.Cu) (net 42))
 (segment (start 105.62999 81.76999) (end 100.09401 81.76999) (width 0.5) (layer F.Cu) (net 42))
 (segment (start 106.68 82.82) (end 105.62999 81.76999) (width 0.5) (layer F.Cu) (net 42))
 (segment (start 101.6 86.70759) (end 101.955011 87.062601) (width 0.25) (layer F.Cu) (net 36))
 (segment (start 101.6 84.82) (end 101.6 86.70759) (width 0.25) (layer F.Cu) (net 36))
 (segment (start 103.762019 98.050979) (end 102.597 99.215998) (width 0.25) (layer F.Cu) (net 36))
 (segment (start 106.127433 98.050979) (end 103.762019 98.050979) (width 0.25) (layer F.Cu) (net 36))
 (segment (start 107.03501 97.143402) (end 106.127433 98.050979) (width 0.25) (layer F.Cu) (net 36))
 (segment (start 107.035011 93.102599) (end 107.03501 97.143402) (width 0.25) (layer F.Cu) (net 36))
 (segment (start 102.597 99.215998) (end 102.597 100.076) (width 0.25) (layer F.Cu) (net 36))
 (segment (start 106.160402 92.22799) (end 107.035011 93.102599) (width 0.25) (layer F.Cu) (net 36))
 (segment (start 101.955011 87.062601) (end 101.955011 90.455201) (width 0.25) (layer F.Cu) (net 36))
 (segment (start 102.827781 91.327971) (end 104.157791 91.327971) (width 0.25) (layer F.Cu) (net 36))
 (segment (start 101.955011 90.455201) (end 102.827781 91.327971) (width 0.25) (layer F.Cu) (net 36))
 (segment (start 104.157791 91.327971) (end 105.03182 92.202) (width 0.25) (layer F.Cu) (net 36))
 (segment (start 105.68999 92.22799) (end 106.160402 92.22799) (width 0.25) (layer F.Cu) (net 36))
 (segment (start 105.664 92.202) (end 105.68999 92.22799) (width 0.25) (layer F.Cu) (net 36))
 (segment (start 105.03182 92.202) (end 105.664 92.202) (width 0.25) (layer F.Cu) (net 36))
 (segment (start 103.251 85.709) (end 104.14 84.82) (width 0.5) (layer F.Cu) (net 41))
 (segment (start 103.251 88.138) (end 103.251 85.709) (width 0.5) (layer F.Cu) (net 41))
 (segment (start 104.14 84.82) (end 106.68 84.82) (width 0.5) (layer F.Cu) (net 41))
 (segment (start 110.509999 85.070001) (end 111.76 83.82) (width 0.5) (layer F.Cu) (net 41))
 (segment (start 106.930001 85.070001) (end 110.509999 85.070001) (width 0.5) (layer F.Cu) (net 41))
 (segment (start 106.68 84.82) (end 106.930001 85.070001) (width 0.5) (layer F.Cu) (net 41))
 (segment (start 109.474 81.28) (end 111.76 81.28) (width 1) (layer F.Cu) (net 1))
 (segment (start 109.474 86.36) (end 111.76 86.36) (width 0.5) (layer F.Cu) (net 5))
 (segment (start 111.76 91.44) (end 109.474 91.44) (width 0.5) (layer F.Cu) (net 9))
 (segment (start 111.76 93.98) (end 109.474 93.98) (width 0.5) (layer F.Cu) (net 11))
 (segment (start 96.52 93.98) (end 94.234 93.98) (width 0.5) (layer F.Cu) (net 18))
 (segment (start 96.52 88.9) (end 94.234 88.9) (width 0.5) (layer F.Cu) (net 22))
 (segment (start 94.234 86.36) (end 96.52 86.36) (width 0.5) (layer F.Cu) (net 24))
 (segment (start 94.234 83.82) (end 96.52 83.82) (width 0.5) (layer F.Cu) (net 26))
 (segment (start 94.234 81.28) (end 96.52 81.28) (width 0.5) (layer F.Cu) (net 28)))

